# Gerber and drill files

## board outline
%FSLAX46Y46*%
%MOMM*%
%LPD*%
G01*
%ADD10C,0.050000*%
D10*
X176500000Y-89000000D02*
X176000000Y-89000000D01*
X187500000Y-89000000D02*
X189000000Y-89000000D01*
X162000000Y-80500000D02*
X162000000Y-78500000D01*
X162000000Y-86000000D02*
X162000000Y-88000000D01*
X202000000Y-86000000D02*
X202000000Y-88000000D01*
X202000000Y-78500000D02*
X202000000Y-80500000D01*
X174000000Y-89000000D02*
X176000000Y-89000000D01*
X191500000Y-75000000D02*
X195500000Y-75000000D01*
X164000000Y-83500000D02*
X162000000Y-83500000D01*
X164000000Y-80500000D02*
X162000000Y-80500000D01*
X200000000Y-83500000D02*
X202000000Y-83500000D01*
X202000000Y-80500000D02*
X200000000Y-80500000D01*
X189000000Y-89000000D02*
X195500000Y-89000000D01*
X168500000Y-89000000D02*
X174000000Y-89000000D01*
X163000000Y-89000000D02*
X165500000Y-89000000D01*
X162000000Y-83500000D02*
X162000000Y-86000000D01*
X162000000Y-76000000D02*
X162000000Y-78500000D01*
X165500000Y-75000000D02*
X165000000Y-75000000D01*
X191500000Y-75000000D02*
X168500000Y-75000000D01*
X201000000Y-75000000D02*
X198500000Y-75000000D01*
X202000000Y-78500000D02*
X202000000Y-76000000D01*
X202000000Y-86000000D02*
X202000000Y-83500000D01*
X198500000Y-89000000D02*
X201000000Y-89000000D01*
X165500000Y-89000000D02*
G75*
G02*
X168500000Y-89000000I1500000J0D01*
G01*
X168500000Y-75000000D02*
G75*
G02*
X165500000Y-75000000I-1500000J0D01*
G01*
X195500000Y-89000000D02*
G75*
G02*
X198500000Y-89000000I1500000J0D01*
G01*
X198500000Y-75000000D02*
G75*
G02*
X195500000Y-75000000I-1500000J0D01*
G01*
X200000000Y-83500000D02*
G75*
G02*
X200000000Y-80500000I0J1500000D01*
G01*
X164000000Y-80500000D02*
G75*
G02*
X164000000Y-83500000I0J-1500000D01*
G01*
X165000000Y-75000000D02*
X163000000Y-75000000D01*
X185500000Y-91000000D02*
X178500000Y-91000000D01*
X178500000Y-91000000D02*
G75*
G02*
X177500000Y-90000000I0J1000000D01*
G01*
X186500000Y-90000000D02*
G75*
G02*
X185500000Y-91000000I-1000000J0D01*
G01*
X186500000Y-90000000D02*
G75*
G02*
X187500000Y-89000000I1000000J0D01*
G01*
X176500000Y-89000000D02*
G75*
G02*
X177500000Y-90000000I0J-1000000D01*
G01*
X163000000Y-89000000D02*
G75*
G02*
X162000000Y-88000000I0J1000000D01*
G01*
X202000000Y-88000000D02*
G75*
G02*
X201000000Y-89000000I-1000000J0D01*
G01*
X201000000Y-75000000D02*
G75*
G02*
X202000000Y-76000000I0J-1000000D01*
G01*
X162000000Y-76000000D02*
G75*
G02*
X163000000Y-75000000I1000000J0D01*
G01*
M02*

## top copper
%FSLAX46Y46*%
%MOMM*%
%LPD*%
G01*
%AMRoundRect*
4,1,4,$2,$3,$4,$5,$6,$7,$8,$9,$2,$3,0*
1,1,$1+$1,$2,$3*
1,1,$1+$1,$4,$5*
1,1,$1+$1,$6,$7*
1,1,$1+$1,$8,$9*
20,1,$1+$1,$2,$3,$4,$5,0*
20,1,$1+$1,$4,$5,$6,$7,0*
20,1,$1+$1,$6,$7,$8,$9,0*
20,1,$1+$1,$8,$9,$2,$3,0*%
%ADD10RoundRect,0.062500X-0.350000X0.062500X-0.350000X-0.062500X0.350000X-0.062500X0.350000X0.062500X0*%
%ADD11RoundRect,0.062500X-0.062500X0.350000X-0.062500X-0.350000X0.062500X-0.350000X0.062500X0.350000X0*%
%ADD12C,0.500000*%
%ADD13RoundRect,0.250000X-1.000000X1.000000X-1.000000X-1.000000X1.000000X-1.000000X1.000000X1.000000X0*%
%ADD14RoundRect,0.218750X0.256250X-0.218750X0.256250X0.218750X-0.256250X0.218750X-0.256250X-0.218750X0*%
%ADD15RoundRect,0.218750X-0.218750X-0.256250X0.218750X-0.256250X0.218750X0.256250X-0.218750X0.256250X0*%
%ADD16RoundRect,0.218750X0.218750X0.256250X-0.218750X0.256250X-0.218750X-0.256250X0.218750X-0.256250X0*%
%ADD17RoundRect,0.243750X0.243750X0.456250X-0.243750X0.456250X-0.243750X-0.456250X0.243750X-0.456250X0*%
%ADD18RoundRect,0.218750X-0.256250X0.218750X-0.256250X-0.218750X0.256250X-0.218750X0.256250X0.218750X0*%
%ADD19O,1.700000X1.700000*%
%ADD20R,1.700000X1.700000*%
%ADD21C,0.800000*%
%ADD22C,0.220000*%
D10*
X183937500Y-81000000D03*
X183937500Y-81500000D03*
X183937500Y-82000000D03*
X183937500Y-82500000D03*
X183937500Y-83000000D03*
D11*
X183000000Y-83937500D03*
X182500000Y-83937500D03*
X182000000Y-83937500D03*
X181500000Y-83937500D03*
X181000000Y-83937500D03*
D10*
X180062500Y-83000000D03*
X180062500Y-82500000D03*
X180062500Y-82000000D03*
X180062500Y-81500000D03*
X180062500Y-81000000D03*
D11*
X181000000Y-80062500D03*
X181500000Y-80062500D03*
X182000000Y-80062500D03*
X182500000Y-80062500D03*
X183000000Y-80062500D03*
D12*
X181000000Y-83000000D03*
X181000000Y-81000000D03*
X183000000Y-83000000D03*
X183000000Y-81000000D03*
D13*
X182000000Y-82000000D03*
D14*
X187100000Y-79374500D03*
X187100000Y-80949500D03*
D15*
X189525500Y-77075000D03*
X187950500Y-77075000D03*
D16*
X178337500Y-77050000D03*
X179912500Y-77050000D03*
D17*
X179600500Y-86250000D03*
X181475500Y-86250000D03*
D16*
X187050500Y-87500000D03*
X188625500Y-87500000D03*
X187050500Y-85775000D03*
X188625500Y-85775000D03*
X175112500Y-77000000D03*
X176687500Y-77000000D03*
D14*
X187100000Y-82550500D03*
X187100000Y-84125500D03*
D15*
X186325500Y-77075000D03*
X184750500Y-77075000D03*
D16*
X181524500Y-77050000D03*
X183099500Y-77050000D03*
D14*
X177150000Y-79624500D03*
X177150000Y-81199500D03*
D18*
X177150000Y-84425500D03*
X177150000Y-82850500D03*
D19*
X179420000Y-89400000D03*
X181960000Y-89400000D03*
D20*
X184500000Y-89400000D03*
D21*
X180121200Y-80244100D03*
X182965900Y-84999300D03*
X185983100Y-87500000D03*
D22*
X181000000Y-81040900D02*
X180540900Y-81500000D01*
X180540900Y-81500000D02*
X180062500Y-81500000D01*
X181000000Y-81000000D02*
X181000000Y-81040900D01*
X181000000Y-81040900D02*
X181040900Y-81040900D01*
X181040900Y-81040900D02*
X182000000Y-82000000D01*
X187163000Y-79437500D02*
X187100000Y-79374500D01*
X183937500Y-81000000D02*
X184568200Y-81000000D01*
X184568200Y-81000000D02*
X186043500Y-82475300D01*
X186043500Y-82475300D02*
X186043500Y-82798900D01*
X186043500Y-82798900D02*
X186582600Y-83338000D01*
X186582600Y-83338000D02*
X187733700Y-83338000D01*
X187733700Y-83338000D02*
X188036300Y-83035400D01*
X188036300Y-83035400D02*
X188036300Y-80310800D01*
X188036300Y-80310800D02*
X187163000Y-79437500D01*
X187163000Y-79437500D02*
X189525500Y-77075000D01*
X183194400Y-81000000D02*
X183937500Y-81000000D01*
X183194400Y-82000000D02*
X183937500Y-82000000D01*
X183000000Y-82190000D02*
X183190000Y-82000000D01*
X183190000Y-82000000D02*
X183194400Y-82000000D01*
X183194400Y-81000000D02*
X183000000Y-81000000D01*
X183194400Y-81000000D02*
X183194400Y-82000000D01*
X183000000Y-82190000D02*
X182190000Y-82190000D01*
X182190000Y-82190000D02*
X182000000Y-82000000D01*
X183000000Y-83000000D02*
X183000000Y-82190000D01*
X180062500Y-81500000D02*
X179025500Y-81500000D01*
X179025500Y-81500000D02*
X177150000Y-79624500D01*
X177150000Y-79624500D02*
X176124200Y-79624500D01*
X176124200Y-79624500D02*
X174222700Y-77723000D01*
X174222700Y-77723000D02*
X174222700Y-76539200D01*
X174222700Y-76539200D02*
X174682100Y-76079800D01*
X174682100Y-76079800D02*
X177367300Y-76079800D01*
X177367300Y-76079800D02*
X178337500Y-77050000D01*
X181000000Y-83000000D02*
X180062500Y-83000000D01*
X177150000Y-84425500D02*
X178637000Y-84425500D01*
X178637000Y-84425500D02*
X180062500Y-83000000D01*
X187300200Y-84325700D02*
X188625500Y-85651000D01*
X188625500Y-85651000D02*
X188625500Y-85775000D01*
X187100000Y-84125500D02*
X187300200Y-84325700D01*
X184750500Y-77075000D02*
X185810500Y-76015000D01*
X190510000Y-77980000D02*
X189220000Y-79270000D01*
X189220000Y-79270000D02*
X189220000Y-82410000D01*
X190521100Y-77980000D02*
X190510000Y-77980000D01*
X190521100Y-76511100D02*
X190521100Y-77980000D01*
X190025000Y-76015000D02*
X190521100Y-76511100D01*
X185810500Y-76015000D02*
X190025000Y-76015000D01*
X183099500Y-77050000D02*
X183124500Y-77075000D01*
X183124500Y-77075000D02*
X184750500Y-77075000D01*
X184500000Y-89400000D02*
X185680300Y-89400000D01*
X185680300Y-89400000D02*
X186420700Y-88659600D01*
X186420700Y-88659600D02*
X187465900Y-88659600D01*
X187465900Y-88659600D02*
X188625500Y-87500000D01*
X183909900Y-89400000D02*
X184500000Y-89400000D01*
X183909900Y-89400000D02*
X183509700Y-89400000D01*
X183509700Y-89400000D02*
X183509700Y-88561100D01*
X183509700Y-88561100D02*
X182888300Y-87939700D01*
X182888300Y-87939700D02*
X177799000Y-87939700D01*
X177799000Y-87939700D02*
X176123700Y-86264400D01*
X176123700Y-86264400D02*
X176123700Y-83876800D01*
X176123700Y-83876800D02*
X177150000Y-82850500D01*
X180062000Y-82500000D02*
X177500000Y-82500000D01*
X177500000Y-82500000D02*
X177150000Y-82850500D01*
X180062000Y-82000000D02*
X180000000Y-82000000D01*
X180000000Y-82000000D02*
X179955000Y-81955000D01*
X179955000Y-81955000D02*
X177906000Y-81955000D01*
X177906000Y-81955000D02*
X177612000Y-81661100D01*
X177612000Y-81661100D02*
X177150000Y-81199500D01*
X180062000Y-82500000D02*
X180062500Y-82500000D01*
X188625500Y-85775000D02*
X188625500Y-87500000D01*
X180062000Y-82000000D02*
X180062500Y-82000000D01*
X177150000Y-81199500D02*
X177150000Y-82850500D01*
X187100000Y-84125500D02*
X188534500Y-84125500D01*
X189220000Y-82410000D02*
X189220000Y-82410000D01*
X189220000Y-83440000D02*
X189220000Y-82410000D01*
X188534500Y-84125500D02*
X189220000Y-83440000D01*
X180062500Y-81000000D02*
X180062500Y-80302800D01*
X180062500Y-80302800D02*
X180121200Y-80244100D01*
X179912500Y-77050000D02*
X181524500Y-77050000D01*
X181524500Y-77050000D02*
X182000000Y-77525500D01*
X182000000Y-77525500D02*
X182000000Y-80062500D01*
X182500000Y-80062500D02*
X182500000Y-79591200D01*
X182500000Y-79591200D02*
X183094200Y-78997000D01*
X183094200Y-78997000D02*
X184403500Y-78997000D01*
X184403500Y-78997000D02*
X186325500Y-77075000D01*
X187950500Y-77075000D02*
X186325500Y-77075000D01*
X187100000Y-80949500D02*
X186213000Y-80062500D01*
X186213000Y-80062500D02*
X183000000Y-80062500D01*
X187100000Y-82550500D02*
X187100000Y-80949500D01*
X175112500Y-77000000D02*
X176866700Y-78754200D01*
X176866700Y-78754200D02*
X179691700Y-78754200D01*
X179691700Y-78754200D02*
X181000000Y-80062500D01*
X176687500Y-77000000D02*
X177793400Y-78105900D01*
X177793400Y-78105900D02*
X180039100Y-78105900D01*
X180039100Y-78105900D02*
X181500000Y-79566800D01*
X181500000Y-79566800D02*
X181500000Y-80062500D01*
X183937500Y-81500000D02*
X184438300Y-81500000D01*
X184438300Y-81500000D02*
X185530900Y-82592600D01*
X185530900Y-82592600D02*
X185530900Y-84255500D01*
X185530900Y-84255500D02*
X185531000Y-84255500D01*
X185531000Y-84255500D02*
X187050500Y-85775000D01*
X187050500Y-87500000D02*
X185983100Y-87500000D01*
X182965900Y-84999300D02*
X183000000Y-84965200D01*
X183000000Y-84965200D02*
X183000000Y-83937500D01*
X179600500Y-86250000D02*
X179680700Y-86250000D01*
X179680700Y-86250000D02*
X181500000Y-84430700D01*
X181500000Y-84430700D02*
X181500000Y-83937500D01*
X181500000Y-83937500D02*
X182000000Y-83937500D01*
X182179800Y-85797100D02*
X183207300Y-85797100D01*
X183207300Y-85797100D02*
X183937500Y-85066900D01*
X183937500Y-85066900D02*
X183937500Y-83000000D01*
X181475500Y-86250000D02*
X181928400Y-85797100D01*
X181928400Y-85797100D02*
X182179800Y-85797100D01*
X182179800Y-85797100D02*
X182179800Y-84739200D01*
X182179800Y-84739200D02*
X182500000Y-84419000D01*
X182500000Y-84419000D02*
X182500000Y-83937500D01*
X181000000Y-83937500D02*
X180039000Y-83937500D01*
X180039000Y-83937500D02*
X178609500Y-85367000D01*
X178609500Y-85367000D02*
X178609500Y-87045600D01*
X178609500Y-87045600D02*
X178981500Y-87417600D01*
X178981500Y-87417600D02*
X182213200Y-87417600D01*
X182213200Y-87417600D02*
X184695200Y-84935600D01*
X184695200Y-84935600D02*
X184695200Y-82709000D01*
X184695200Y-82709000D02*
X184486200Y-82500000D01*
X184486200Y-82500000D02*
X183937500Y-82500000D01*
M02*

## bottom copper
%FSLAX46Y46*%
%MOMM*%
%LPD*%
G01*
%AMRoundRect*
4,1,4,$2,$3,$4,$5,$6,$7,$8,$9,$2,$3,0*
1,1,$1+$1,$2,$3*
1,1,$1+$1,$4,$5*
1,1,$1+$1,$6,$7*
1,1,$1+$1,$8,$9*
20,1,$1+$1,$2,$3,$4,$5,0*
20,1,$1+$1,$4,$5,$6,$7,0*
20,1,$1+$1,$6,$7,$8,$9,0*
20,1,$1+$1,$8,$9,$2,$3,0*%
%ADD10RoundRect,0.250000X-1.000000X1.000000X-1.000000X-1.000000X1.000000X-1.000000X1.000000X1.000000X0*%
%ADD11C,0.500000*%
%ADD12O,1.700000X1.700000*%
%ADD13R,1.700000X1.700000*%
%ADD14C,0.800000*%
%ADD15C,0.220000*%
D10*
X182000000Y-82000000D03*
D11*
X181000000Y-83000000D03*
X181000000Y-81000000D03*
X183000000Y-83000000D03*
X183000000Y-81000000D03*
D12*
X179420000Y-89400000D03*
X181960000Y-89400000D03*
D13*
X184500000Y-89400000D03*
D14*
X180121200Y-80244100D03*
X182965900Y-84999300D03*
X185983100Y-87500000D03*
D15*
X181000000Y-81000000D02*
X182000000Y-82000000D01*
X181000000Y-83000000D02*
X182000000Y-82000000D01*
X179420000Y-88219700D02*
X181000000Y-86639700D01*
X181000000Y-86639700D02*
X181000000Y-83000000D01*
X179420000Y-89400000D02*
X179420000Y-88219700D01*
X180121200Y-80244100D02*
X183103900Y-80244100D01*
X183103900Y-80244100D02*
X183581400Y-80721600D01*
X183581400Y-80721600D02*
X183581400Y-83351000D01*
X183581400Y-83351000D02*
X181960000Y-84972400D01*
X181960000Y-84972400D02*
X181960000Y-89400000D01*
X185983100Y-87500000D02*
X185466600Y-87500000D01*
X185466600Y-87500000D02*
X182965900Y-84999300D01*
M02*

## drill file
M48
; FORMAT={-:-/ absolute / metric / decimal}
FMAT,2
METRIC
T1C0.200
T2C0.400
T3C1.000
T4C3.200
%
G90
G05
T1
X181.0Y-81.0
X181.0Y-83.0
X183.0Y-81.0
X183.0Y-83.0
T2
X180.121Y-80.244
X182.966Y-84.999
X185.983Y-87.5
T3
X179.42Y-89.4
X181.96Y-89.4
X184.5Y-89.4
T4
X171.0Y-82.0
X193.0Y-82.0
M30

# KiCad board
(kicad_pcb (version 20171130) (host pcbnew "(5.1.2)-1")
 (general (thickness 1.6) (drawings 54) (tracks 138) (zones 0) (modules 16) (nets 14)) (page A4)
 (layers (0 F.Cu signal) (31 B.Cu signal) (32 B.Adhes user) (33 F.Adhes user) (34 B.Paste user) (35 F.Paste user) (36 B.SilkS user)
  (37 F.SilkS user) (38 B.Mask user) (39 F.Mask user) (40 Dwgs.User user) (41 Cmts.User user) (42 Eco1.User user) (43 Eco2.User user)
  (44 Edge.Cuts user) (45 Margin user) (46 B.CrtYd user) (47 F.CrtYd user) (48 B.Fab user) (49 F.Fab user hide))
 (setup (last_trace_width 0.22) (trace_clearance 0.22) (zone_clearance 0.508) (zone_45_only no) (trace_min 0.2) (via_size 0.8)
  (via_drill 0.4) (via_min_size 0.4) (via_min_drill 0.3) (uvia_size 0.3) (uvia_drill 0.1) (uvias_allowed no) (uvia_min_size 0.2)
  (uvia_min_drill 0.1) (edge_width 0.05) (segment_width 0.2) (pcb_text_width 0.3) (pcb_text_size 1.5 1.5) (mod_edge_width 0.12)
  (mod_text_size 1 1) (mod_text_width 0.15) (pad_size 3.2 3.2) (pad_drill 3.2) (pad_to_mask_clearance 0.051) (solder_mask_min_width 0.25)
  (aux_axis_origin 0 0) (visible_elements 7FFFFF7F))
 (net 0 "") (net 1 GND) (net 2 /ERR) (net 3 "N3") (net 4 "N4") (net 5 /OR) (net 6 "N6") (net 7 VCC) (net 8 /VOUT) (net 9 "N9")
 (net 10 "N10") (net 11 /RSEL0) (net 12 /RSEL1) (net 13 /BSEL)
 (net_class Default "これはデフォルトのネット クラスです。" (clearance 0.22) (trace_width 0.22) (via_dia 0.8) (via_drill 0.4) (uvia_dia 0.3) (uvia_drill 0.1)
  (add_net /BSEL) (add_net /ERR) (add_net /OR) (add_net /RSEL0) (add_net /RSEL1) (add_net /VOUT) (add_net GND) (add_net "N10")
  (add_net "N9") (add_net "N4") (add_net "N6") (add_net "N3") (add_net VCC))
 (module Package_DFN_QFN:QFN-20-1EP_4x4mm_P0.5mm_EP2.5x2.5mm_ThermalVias (layer F.Cu) (at 182 82 270)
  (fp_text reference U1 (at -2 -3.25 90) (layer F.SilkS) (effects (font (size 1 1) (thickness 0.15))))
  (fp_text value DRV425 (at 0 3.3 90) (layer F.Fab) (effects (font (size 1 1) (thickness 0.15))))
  (pad 20 smd roundrect (at -1 -1.9375 270) (size 0.25 0.825) (layers F.Cu F.Paste F.Mask) (roundrect_rratio 0.25) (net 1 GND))
  (pad 19 smd roundrect (at -0.5 -1.9375 270) (size 0.25 0.825) (layers F.Cu F.Paste F.Mask) (roundrect_rratio 0.25) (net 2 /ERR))
  (pad 18 smd roundrect (at 0 -1.9375 270) (size 0.25 0.825) (layers F.Cu F.Paste F.Mask) (roundrect_rratio 0.25) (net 1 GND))
  (pad 17 smd roundrect (at 0.5 -1.9375 270) (size 0.25 0.825) (layers F.Cu F.Paste F.Mask) (roundrect_rratio 0.25) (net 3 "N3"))
  (pad 16 smd roundrect (at 1 -1.9375 270) (size 0.25 0.825) (layers F.Cu F.Paste F.Mask) (roundrect_rratio 0.25) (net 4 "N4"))
  (pad 15 smd roundrect (at 1.9375 -1 270) (size 0.825 0.25) (layers F.Cu F.Paste F.Mask) (roundrect_rratio 0.25) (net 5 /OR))
  (pad 14 smd roundrect (at 1.9375 -0.5 270) (size 0.825 0.25) (layers F.Cu F.Paste F.Mask) (roundrect_rratio 0.25) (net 4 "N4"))
  (pad 13 smd roundrect (at 1.9375 0 270) (size 0.825 0.25) (layers F.Cu F.Paste F.Mask) (roundrect_rratio 0.25) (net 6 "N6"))
  (pad 12 smd roundrect (at 1.9375 0.5 270) (size 0.825 0.25) (layers F.Cu F.Paste F.Mask) (roundrect_rratio 0.25) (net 6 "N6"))
  (pad 11 smd roundrect (at 1.9375 1 270) (size 0.825 0.25) (layers F.Cu F.Paste F.Mask) (roundrect_rratio 0.25) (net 3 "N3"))
  (pad 10 smd roundrect (at 1 1.9375 270) (size 0.25 0.825) (layers F.Cu F.Paste F.Mask) (roundrect_rratio 0.25) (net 1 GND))
  (pad 9 smd roundrect (at 0.5 1.9375 270) (size 0.25 0.825) (layers F.Cu F.Paste F.Mask) (roundrect_rratio 0.25) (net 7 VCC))
  (pad 8 smd roundrect (at 0 1.9375 270) (size 0.25 0.825) (layers F.Cu F.Paste F.Mask) (roundrect_rratio 0.25) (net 7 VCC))
  (pad 7 smd roundrect (at -0.5 1.9375 270) (size 0.25 0.825) (layers F.Cu F.Paste F.Mask) (roundrect_rratio 0.25) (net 1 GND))
  (pad 6 smd roundrect (at -1 1.9375 270) (size 0.25 0.825) (layers F.Cu F.Paste F.Mask) (roundrect_rratio 0.25) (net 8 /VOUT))
  (pad 5 smd roundrect (at -1.9375 1 270) (size 0.825 0.25) (layers F.Cu F.Paste F.Mask) (roundrect_rratio 0.25) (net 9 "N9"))
  (pad 4 smd roundrect (at -1.9375 0.5 270) (size 0.825 0.25) (layers F.Cu F.Paste F.Mask) (roundrect_rratio 0.25) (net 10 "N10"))
  (pad 3 smd roundrect (at -1.9375 0 270) (size 0.825 0.25) (layers F.Cu F.Paste F.Mask) (roundrect_rratio 0.25) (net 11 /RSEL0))
  (pad 2 smd roundrect (at -1.9375 -0.5 270) (size 0.825 0.25) (layers F.Cu F.Paste F.Mask) (roundrect_rratio 0.25) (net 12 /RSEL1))
  (pad 1 smd roundrect (at -1.9375 -1 270) (size 0.825 0.25) (layers F.Cu F.Paste F.Mask) (roundrect_rratio 0.25) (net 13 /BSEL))
  (pad "" smd roundrect (at 0.625 0.625 270) (size 1.08 1.08) (layers F.Paste) (roundrect_rratio 0.231481))
  (pad "" smd roundrect (at 0.625 -0.625 270) (size 1.08 1.08) (layers F.Paste) (roundrect_rratio 0.231481))
  (pad "" smd roundrect (at -0.625 0.625 270) (size 1.08 1.08) (layers F.Paste) (roundrect_rratio 0.231481))
  (pad "" smd roundrect (at -0.625 -0.625 270) (size 1.08 1.08) (layers F.Paste) (roundrect_rratio 0.231481))
  (pad 21 smd roundrect (at 0 0 270) (size 2.5 2.5) (layers B.Cu) (roundrect_rratio 0.1) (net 1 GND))
  (pad 21 thru_hole circle (at 1 1 270) (size 0.5 0.5) (drill 0.2) (layers *.Cu) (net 1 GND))
  (pad 21 thru_hole circle (at -1 1 270) (size 0.5 0.5) (drill 0.2) (layers *.Cu) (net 1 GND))
  (pad 21 thru_hole circle (at 1 -1 270) (size 0.5 0.5) (drill 0.2) (layers *.Cu) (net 1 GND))
  (pad 21 thru_hole circle (at -1 -1 270) (size 0.5 0.5) (drill 0.2) (layers *.Cu) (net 1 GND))
  (pad 21 smd roundrect (at 0 0 270) (size 2.5 2.5) (layers F.Cu F.Mask) (roundrect_rratio 0.1) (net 1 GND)))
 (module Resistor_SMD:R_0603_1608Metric (layer F.Cu) (at 187.1 80.162 90)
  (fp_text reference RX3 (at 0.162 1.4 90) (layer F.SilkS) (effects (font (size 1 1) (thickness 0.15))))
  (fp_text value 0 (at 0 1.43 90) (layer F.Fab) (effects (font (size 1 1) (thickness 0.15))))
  (pad 2 smd roundrect (at 0.7875 0 90) (size 0.875 0.95) (layers F.Cu F.Paste F.Mask) (roundrect_rratio 0.25) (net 1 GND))
  (pad 1 smd roundrect (at -0.7875 0 90) (size 0.875 0.95) (layers F.Cu F.Paste F.Mask) (roundrect_rratio 0.25) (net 13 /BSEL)))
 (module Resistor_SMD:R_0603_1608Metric (layer F.Cu) (at 188.738 77.075)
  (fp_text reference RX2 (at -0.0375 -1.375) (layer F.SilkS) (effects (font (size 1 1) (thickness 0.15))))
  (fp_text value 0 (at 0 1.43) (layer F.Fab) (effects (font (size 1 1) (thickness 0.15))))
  (pad 2 smd roundrect (at 0.7875 0) (size 0.875 0.95) (layers F.Cu F.Paste F.Mask) (roundrect_rratio 0.25) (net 1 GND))
  (pad 1 smd roundrect (at -0.7875 0) (size 0.875 0.95) (layers F.Cu F.Paste F.Mask) (roundrect_rratio 0.25) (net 12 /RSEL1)))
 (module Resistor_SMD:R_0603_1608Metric (layer F.Cu) (at 179.125 77.05 180)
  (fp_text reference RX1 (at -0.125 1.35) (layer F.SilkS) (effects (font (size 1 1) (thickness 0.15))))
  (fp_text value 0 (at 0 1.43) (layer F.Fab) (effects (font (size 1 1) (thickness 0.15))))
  (pad 2 smd roundrect (at 0.7875 0 180) (size 0.875 0.95) (layers F.Cu F.Paste F.Mask) (roundrect_rratio 0.25) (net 1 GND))
  (pad 1 smd roundrect (at -0.7875 0 180) (size 0.875 0.95) (layers F.Cu F.Paste F.Mask) (roundrect_rratio 0.25) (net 11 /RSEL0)))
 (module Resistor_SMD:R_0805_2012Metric (layer F.Cu) (at 180.538 86.25 180)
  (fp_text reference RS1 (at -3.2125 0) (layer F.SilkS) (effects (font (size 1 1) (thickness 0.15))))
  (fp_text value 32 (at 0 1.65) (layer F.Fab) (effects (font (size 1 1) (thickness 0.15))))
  (pad 2 smd roundrect (at 0.9375 0 180) (size 0.975 1.4) (layers F.Cu F.Paste F.Mask) (roundrect_rratio 0.25) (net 6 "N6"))
  (pad 1 smd roundrect (at -0.9375 0 180) (size 0.975 1.4) (layers F.Cu F.Paste F.Mask) (roundrect_rratio 0.25) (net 4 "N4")))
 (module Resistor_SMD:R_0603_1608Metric (layer F.Cu) (at 187.838 87.5 180)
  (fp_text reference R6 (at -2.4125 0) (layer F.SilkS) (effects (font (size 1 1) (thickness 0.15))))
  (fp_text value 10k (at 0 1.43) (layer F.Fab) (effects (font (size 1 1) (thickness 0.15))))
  (pad 2 smd roundrect (at 0.7875 0 180) (size 0.875 0.95) (layers F.Cu F.Paste F.Mask) (roundrect_rratio 0.25) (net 5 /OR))
  (pad 1 smd roundrect (at -0.7875 0 180) (size 0.875 0.95) (layers F.Cu F.Paste F.Mask) (roundrect_rratio 0.25) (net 7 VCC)))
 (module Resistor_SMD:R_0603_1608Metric (layer F.Cu) (at 187.838 85.775 180)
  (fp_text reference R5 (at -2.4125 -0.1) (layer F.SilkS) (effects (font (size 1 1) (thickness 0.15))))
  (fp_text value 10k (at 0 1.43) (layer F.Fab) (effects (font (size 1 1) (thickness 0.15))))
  (pad 2 smd roundrect (at 0.7875 0 180) (size 0.875 0.95) (layers F.Cu F.Paste F.Mask) (roundrect_rratio 0.25) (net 2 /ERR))
  (pad 1 smd roundrect (at -0.7875 0 180) (size 0.875 0.95) (layers F.Cu F.Paste F.Mask) (roundrect_rratio 0.25) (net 7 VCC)))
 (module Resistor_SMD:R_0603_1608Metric (layer F.Cu) (at 175.9 77 180)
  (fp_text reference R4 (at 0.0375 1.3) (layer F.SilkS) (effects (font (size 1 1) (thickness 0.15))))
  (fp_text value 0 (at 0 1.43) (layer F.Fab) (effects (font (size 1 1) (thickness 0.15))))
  (pad 2 smd roundrect (at 0.7875 0 180) (size 0.875 0.95) (layers F.Cu F.Paste F.Mask) (roundrect_rratio 0.25) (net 9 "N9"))
  (pad 1 smd roundrect (at -0.7875 0 180) (size 0.875 0.95) (layers F.Cu F.Paste F.Mask) (roundrect_rratio 0.25) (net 10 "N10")))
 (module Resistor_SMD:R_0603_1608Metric (layer F.Cu) (at 187.1 83.338 90)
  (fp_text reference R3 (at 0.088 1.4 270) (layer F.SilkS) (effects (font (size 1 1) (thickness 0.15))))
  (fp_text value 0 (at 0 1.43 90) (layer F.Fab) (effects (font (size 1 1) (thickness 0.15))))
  (pad 2 smd roundrect (at 0.7875 0 90) (size 0.875 0.95) (layers F.Cu F.Paste F.Mask) (roundrect_rratio 0.25) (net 13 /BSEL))
  (pad 1 smd roundrect (at -0.7875 0 90) (size 0.875 0.95) (layers F.Cu F.Paste F.Mask) (roundrect_rratio 0.25) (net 7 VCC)))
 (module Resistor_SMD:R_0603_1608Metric (layer F.Cu) (at 185.538 77.075)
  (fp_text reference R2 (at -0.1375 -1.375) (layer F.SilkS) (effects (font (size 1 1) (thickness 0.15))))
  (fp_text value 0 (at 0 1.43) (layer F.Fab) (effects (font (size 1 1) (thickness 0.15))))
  (pad 2 smd roundrect (at 0.7875 0) (size 0.875 0.95) (layers F.Cu F.Paste F.Mask) (roundrect_rratio 0.25) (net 12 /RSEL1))
  (pad 1 smd roundrect (at -0.7875 0) (size 0.875 0.95) (layers F.Cu F.Paste F.Mask) (roundrect_rratio 0.25) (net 7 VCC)))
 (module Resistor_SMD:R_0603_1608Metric (layer F.Cu) (at 182.312 77.05 180)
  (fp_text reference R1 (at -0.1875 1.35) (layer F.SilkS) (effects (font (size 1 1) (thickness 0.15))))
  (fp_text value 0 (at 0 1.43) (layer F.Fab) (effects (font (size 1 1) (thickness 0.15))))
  (pad 2 smd roundrect (at 0.7875 0 180) (size 0.875 0.95) (layers F.Cu F.Paste F.Mask) (roundrect_rratio 0.25) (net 11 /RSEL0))
  (pad 1 smd roundrect (at -0.7875 0 180) (size 0.875 0.95) (layers F.Cu F.Paste F.Mask) (roundrect_rratio 0.25) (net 7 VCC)))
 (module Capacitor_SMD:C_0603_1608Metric (layer F.Cu) (at 177.15 80.412 90)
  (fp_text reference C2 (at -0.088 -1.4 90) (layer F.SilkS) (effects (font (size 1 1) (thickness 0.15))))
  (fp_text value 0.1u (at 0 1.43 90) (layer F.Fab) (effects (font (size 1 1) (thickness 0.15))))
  (pad 2 smd roundrect (at 0.7875 0 90) (size 0.875 0.95) (layers F.Cu F.Paste F.Mask) (roundrect_rratio 0.25) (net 1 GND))
  (pad 1 smd roundrect (at -0.7875 0 90) (size 0.875 0.95) (layers F.Cu F.Paste F.Mask) (roundrect_rratio 0.25) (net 7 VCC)))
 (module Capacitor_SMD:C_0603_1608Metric (layer F.Cu) (at 177.15 83.638 270)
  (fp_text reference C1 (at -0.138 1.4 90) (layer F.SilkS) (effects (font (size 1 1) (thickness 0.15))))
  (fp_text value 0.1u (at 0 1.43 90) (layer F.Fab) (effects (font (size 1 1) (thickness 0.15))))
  (pad 2 smd roundrect (at 0.7875 0 270) (size 0.875 0.95) (layers F.Cu F.Paste F.Mask) (roundrect_rratio 0.25) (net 1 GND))
  (pad 1 smd roundrect (at -0.7875 0 270) (size 0.875 0.95) (layers F.Cu F.Paste F.Mask) (roundrect_rratio 0.25) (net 7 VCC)))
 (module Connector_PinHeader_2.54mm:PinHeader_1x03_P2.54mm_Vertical (layer F.Cu) (at 184.5 89.4 270)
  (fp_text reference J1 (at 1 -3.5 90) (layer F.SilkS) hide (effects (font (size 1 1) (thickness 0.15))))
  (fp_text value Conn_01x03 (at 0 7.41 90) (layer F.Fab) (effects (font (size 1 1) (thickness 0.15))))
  (pad 3 thru_hole oval (at 0 5.08 270) (size 1.7 1.7) (drill 1) (layers *.Cu *.Mask) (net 1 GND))
  (pad 2 thru_hole oval (at 0 2.54 270) (size 1.7 1.7) (drill 1) (layers *.Cu *.Mask) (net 8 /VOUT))
  (pad 1 thru_hole rect (at 0 0 270) (size 1.7 1.7) (drill 1) (layers *.Cu *.Mask) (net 7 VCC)))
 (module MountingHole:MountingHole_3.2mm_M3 (layer F.Cu) (at 171 82)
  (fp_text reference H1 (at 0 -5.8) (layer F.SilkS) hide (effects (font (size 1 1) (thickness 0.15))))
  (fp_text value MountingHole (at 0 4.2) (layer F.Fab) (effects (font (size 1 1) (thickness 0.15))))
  (pad "" np_thru_hole circle (at 0 0) (size 3.2 3.2) (drill 3.2) (layers *.Cu)))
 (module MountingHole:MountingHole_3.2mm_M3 (layer F.Cu) (at 193 82)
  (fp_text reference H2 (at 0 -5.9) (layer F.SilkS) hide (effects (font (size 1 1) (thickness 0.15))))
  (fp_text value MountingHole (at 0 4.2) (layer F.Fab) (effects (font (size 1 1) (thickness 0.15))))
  (pad "" np_thru_hole circle (at 0 0) (size 3.2 3.2) (drill 3.2) (layers *.Cu)))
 (gr_line (start 176.5 89) (end 176 89) (layer Edge.Cuts) (width 0.05))
 (gr_line (start 187.5 89) (end 189 89) (layer Edge.Cuts) (width 0.05))
 (gr_line (start 162 80.5) (end 162 78.5) (layer Edge.Cuts) (width 0.05))
 (gr_line (start 162 86) (end 162 88) (layer Edge.Cuts) (width 0.05))
 (gr_line (start 202 86) (end 202 88) (layer Edge.Cuts) (width 0.05))
 (gr_line (start 202 78.5) (end 202 80.5) (layer Edge.Cuts) (width 0.05))
 (gr_line (start 174 89) (end 176 89) (layer Edge.Cuts) (width 0.05))
 (gr_line (start 191.5 75) (end 195.5 75) (layer Edge.Cuts) (width 0.05))
 (gr_line (start 164 83.5) (end 162 83.5) (layer Edge.Cuts) (width 0.05))
 (gr_line (start 164 80.5) (end 162 80.5) (layer Edge.Cuts) (width 0.05))
 (gr_line (start 200 83.5) (end 202 83.5) (layer Edge.Cuts) (width 0.05))
 (gr_line (start 202 80.5) (end 200 80.5) (layer Edge.Cuts) (width 0.05))
 (gr_line (start 189 89) (end 195.5 89) (layer Edge.Cuts) (width 0.05))
 (gr_line (start 168.5 89) (end 174 89) (layer Edge.Cuts) (width 0.05))
 (gr_line (start 163 89) (end 165.5 89) (layer Edge.Cuts) (width 0.05))
 (gr_line (start 162 83.5) (end 162 86) (layer Edge.Cuts) (width 0.05))
 (gr_line (start 162 76) (end 162 78.5) (layer Edge.Cuts) (width 0.05))
 (gr_line (start 165.5 75) (end 165 75) (layer Edge.Cuts) (width 0.05))
 (gr_line (start 191.5 75) (end 168.5 75) (layer Edge.Cuts) (width 0.05))
 (gr_line (start 201 75) (end 198.5 75) (layer Edge.Cuts) (width 0.05))
 (gr_line (start 202 78.5) (end 202 76) (layer Edge.Cuts) (width 0.05))
 (gr_line (start 202 86) (end 202 83.5) (layer Edge.Cuts) (width 0.05))
 (gr_line (start 198.5 89) (end 201 89) (layer Edge.Cuts) (width 0.05))
 (gr_arc (start 167 89) (end 168.5 89) (angle -180) (layer Edge.Cuts) (width 0.05))
 (gr_arc (start 167 75) (end 165.5 75) (angle -180) (layer Edge.Cuts) (width 0.05))
 (gr_arc (start 197 89) (end 198.5 89) (angle -180) (layer Edge.Cuts) (width 0.05))
 (gr_arc (start 197 75) (end 195.5 75) (angle -180) (layer Edge.Cuts) (width 0.05))
 (gr_arc (start 200 82) (end 200 80.5) (angle -180) (layer Edge.Cuts) (width 0.05))
 (gr_arc (start 164 82) (end 164 83.5) (angle -180) (layer Edge.Cuts) (width 0.05))
 (gr_line (start 165 75) (end 163 75) (layer Edge.Cuts) (width 0.05))
 (gr_line (start 185.5 91) (end 178.5 91) (layer Edge.Cuts) (width 0.05))
 (gr_arc (start 178.5 90) (end 177.5 90) (angle -90) (layer Edge.Cuts) (width 0.05))
 (gr_arc (start 185.5 90) (end 185.5 91) (angle -90) (layer Edge.Cuts) (width 0.05))
 (gr_arc (start 187.5 90) (end 187.5 89) (angle -90) (layer Edge.Cuts) (width 0.05))
 (gr_arc (start 176.5 90) (end 177.5 90) (angle -90) (layer Edge.Cuts) (width 0.05))
 (gr_arc (start 163 88) (end 162 88) (angle -90) (layer Edge.Cuts) (width 0.05))
 (gr_arc (start 201 88) (end 201 89) (angle -90) (layer Edge.Cuts) (width 0.05))
 (gr_arc (start 201 76) (end 202 76) (angle -90) (layer Edge.Cuts) (width 0.05))
 (gr_arc (start 163 76) (end 163 75) (angle -90) (layer Edge.Cuts) (width 0.05))
 (segment (start 181 81.0409) (end 180.5409 81.5) (width 0.22) (layer F.Cu) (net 1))
 (segment (start 180.5409 81.5) (end 180.0625 81.5) (width 0.22) (layer F.Cu) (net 1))
 (segment (start 181 81) (end 181 81.0409) (width 0.22) (layer F.Cu) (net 1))
 (segment (start 181 81.0409) (end 181.0409 81.0409) (width 0.22) (layer F.Cu) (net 1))
 (segment (start 181.0409 81.0409) (end 182 82) (width 0.22) (layer F.Cu) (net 1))
 (segment (start 187.163 79.4375) (end 187.1 79.3745) (width 0.22) (layer F.Cu) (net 1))
 (segment (start 183.9375 81) (end 184.5682 81) (width 0.22) (layer F.Cu) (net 1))
 (segment (start 184.5682 81) (end 186.0435 82.4753) (width 0.22) (layer F.Cu) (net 1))
 (segment (start 186.0435 82.4753) (end 186.0435 82.7989) (width 0.22) (layer F.Cu) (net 1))
 (segment (start 186.0435 82.7989) (end 186.5826 83.338) (width 0.22) (layer F.Cu) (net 1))
 (segment (start 186.5826 83.338) (end 187.7337 83.338) (width 0.22) (layer F.Cu) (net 1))
 (segment (start 187.7337 83.338) (end 188.0363 83.0354) (width 0.22) (layer F.Cu) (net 1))
 (segment (start 188.0363 83.0354) (end 188.0363 80.3108) (width 0.22) (layer F.Cu) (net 1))
 (segment (start 188.0363 80.3108) (end 187.163 79.4375) (width 0.22) (layer F.Cu) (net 1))
 (segment (start 187.163 79.4375) (end 189.5255 77.075) (width 0.22) (layer F.Cu) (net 1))
 (segment (start 183.1944 81) (end 183.9375 81) (width 0.22) (layer F.Cu) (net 1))
 (segment (start 183.1944 82) (end 183.9375 82) (width 0.22) (layer F.Cu) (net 1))
 (segment (start 183 82.19) (end 183.19 82) (width 0.22) (layer F.Cu) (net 1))
 (segment (start 183.19 82) (end 183.1944 82) (width 0.22) (layer F.Cu) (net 1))
 (segment (start 183.1944 81) (end 183 81) (width 0.22) (layer F.Cu) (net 1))
 (segment (start 183.1944 81) (end 183.1944 82) (width 0.22) (layer F.Cu) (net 1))
 (segment (start 183 82.19) (end 182.19 82.19) (width 0.22) (layer F.Cu) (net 1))
 (segment (start 182.19 82.19) (end 182 82) (width 0.22) (layer F.Cu) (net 1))
 (segment (start 183 83) (end 183 82.19) (width 0.22) (layer F.Cu) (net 1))
 (segment (start 180.0625 81.5) (end 179.0255 81.5) (width 0.22) (layer F.Cu) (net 1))
 (segment (start 179.0255 81.5) (end 177.15 79.6245) (width 0.22) (layer F.Cu) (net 1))
 (segment (start 177.15 79.6245) (end 176.1242 79.6245) (width 0.22) (layer F.Cu) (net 1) (status 400000))
 (segment (start 176.1242 79.6245) (end 174.2227 77.723) (width 0.22) (layer F.Cu) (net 1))
 (segment (start 174.2227 77.723) (end 174.2227 76.5392) (width 0.22) (layer F.Cu) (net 1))
 (segment (start 174.2227 76.5392) (end 174.6821 76.0798) (width 0.22) (layer F.Cu) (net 1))
 (segment (start 174.6821 76.0798) (end 177.3673 76.0798) (width 0.22) (layer F.Cu) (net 1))
 (segment (start 177.3673 76.0798) (end 178.3375 77.05) (width 0.22) (layer F.Cu) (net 1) (status 800000))
 (segment (start 181 81) (end 182 82) (width 0.22) (layer B.Cu) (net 1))
 (segment (start 181 83) (end 182 82) (width 0.22) (layer B.Cu) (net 1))
 (segment (start 179.42 88.2197) (end 181 86.6397) (width 0.22) (layer B.Cu) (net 1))
 (segment (start 181 86.6397) (end 181 83) (width 0.22) (layer B.Cu) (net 1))
 (segment (start 181 83) (end 180.0625 83) (width 0.22) (layer F.Cu) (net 1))
 (segment (start 177.15 84.4255) (end 178.637 84.4255) (width 0.22) (layer F.Cu) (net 1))
 (segment (start 178.637 84.4255) (end 180.0625 83) (width 0.22) (layer F.Cu) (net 1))
 (segment (start 179.42 89.4) (end 179.42 88.2197) (width 0.22) (layer B.Cu) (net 1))
 (segment (start 187.3002 84.3257) (end 188.6255 85.651) (width 0.22) (layer F.Cu) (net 7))
 (segment (start 188.6255 85.651) (end 188.6255 85.775) (width 0.22) (layer F.Cu) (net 7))
 (segment (start 187.1 84.1255) (end 187.3002 84.3257) (width 0.22) (layer F.Cu) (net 7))
 (segment (start 184.7505 77.075) (end 185.8105 76.015) (width 0.22) (layer F.Cu) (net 7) (status 400000))
 (segment (start 190.51 77.98) (end 189.22 79.27) (width 0.22) (layer F.Cu) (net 7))
 (segment (start 189.22 79.27) (end 189.22 82.41) (width 0.22) (layer F.Cu) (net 7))
 (segment (start 190.5211 77.98) (end 190.51 77.98) (width 0.22) (layer F.Cu) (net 7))
 (segment (start 190.5211 76.5111) (end 190.5211 77.98) (width 0.22) (layer F.Cu) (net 7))
 (segment (start 190.025 76.015) (end 190.5211 76.5111) (width 0.22) (layer F.Cu) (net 7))
 (segment (start 185.8105 76.015) (end 190.025 76.015) (width 0.22) (layer F.Cu) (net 7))
 (segment (start 183.0995 77.05) (end 183.1245 77.075) (width 0.22) (layer F.Cu) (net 7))
 (segment (start 183.1245 77.075) (end 184.7505 77.075) (width 0.22) (layer F.Cu) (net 7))
 (segment (start 184.5 89.4) (end 185.6803 89.4) (width 0.22) (layer F.Cu) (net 7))
 (segment (start 185.6803 89.4) (end 186.4207 88.6596) (width 0.22) (layer F.Cu) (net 7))
 (segment (start 186.4207 88.6596) (end 187.4659 88.6596) (width 0.22) (layer F.Cu) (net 7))
 (segment (start 187.4659 88.6596) (end 188.6255 87.5) (width 0.22) (layer F.Cu) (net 7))
 (segment (start 183.9099 89.4) (end 184.5 89.4) (width 0.22) (layer F.Cu) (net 7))
 (segment (start 183.9099 89.4) (end 183.5097 89.4) (width 0.22) (layer F.Cu) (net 7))
 (segment (start 183.5097 89.4) (end 183.5097 88.5611) (width 0.22) (layer F.Cu) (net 7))
 (segment (start 183.5097 88.5611) (end 182.8883 87.9397) (width 0.22) (layer F.Cu) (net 7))
 (segment (start 182.8883 87.9397) (end 177.799 87.9397) (width 0.22) (layer F.Cu) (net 7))
 (segment (start 177.799 87.9397) (end 176.1237 86.2644) (width 0.22) (layer F.Cu) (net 7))
 (segment (start 176.1237 86.2644) (end 176.1237 83.8768) (width 0.22) (layer F.Cu) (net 7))
 (segment (start 176.1237 83.8768) (end 177.15 82.8505) (width 0.22) (layer F.Cu) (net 7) (status 800000))
 (segment (start 180.062 82.5) (end 177.5 82.5) (width 0.22) (layer F.Cu) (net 7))
 (segment (start 177.5 82.5) (end 177.15 82.8505) (width 0.22) (layer F.Cu) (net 7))
 (segment (start 180.062 82) (end 180 82) (width 0.22) (layer F.Cu) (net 7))
 (segment (start 180 82) (end 179.955 81.955) (width 0.22) (layer F.Cu) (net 7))
 (segment (start 179.955 81.955) (end 177.906 81.955) (width 0.22) (layer F.Cu) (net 7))
 (segment (start 177.906 81.955) (end 177.612 81.6611) (width 0.22) (layer F.Cu) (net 7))
 (segment (start 177.612 81.6611) (end 177.15 81.1995) (width 0.22) (layer F.Cu) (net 7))
 (segment (start 180.062 82.5) (end 180.0625 82.5) (width 0.22) (layer F.Cu) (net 7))
 (segment (start 188.6255 85.775) (end 188.6255 87.5) (width 0.22) (layer F.Cu) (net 7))
 (segment (start 180.062 82) (end 180.0625 82) (width 0.22) (layer F.Cu) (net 7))
 (segment (start 177.15 81.1995) (end 177.15 82.8505) (width 0.22) (layer F.Cu) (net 7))
 (segment (start 187.1 84.1255) (end 188.5345 84.1255) (width 0.22) (layer F.Cu) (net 7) (status 400000))
 (segment (start 189.22 82.41) (end 189.22 82.41) (width 0.22) (layer F.Cu) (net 7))
 (segment (start 189.22 83.44) (end 189.22 82.41) (width 0.22) (layer F.Cu) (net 7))
 (segment (start 188.5345 84.1255) (end 189.22 83.44) (width 0.22) (layer F.Cu) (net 7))
 (segment (start 180.1212 80.2441) (end 183.1039 80.2441) (width 0.22) (layer B.Cu) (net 8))
 (segment (start 183.1039 80.2441) (end 183.5814 80.7216) (width 0.22) (layer B.Cu) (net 8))
 (segment (start 183.5814 80.7216) (end 183.5814 83.351) (width 0.22) (layer B.Cu) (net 8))
 (segment (start 183.5814 83.351) (end 181.96 84.9724) (width 0.22) (layer B.Cu) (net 8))
 (segment (start 181.96 84.9724) (end 181.96 89.4) (width 0.22) (layer B.Cu) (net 8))
 (segment (start 180.0625 81) (end 180.0625 80.3028) (width 0.22) (layer F.Cu) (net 8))
 (segment (start 180.0625 80.3028) (end 180.1212 80.2441) (width 0.22) (layer F.Cu) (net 8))
 (via (at 180.1212 80.2441) (size 0.8) (layers F.Cu B.Cu) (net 8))
 (segment (start 179.9125 77.05) (end 181.5245 77.05) (width 0.22) (layer F.Cu) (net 11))
 (segment (start 181.5245 77.05) (end 182 77.5255) (width 0.22) (layer F.Cu) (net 11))
 (segment (start 182 77.5255) (end 182 80.0625) (width 0.22) (layer F.Cu) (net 11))
 (segment (start 182.5 80.0625) (end 182.5 79.5912) (width 0.22) (layer F.Cu) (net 12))
 (segment (start 182.5 79.5912) (end 183.0942 78.997) (width 0.22) (layer F.Cu) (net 12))
 (segment (start 183.0942 78.997) (end 184.4035 78.997) (width 0.22) (layer F.Cu) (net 12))
 (segment (start 184.4035 78.997) (end 186.3255 77.075) (width 0.22) (layer F.Cu) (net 12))
 (segment (start 187.9505 77.075) (end 186.3255 77.075) (width 0.22) (layer F.Cu) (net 12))
 (segment (start 187.1 80.9495) (end 186.213 80.0625) (width 0.22) (layer F.Cu) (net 13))
 (segment (start 186.213 80.0625) (end 183 80.0625) (width 0.22) (layer F.Cu) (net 13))
 (segment (start 187.1 82.5505) (end 187.1 80.9495) (width 0.22) (layer F.Cu) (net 13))
 (segment (start 175.1125 77) (end 176.8667 78.7542) (width 0.22) (layer F.Cu) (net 9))
 (segment (start 176.8667 78.7542) (end 179.6917 78.7542) (width 0.22) (layer F.Cu) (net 9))
 (segment (start 179.6917 78.7542) (end 181 80.0625) (width 0.22) (layer F.Cu) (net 9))
 (segment (start 176.6875 77) (end 177.7934 78.1059) (width 0.22) (layer F.Cu) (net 10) (status 400000))
 (segment (start 177.7934 78.1059) (end 180.0391 78.1059) (width 0.22) (layer F.Cu) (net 10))
 (segment (start 180.0391 78.1059) (end 181.5 79.5668) (width 0.22) (layer F.Cu) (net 10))
 (segment (start 181.5 79.5668) (end 181.5 80.0625) (width 0.22) (layer F.Cu) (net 10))
 (segment (start 183.9375 81.5) (end 184.4383 81.5) (width 0.22) (layer F.Cu) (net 2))
 (segment (start 184.4383 81.5) (end 185.5309 82.5926) (width 0.22) (layer F.Cu) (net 2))
 (segment (start 185.5309 82.5926) (end 185.5309 84.2555) (width 0.22) (layer F.Cu) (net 2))
 (segment (start 185.5309 84.2555) (end 185.531 84.2555) (width 0.22) (layer F.Cu) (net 2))
 (segment (start 185.531 84.2555) (end 187.0505 85.775) (width 0.22) (layer F.Cu) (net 2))
 (segment (start 187.0505 87.5) (end 185.9831 87.5) (width 0.22) (layer F.Cu) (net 5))
 (segment (start 182.9659 84.9993) (end 183 84.9652) (width 0.22) (layer F.Cu) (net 5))
 (segment (start 183 84.9652) (end 183 83.9375) (width 0.22) (layer F.Cu) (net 5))
 (via (at 182.9659 84.9993) (size 0.8) (layers F.Cu B.Cu) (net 5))
 (via (at 185.9831 87.5) (size 0.8) (layers F.Cu B.Cu) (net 5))
 (segment (start 185.9831 87.5) (end 185.4666 87.5) (width 0.22) (layer B.Cu) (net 5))
 (segment (start 185.4666 87.5) (end 182.9659 84.9993) (width 0.22) (layer B.Cu) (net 5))
 (segment (start 179.6005 86.25) (end 179.6807 86.25) (width 0.22) (layer F.Cu) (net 6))
 (segment (start 179.6807 86.25) (end 181.5 84.4307) (width 0.22) (layer F.Cu) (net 6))
 (segment (start 181.5 84.4307) (end 181.5 83.9375) (width 0.22) (layer F.Cu) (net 6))
 (segment (start 181.5 83.9375) (end 182 83.9375) (width 0.22) (layer F.Cu) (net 6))
 (segment (start 182.1798 85.7971) (end 183.2073 85.7971) (width 0.22) (layer F.Cu) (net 4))
 (segment (start 183.2073 85.7971) (end 183.9375 85.0669) (width 0.22) (layer F.Cu) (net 4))
 (segment (start 183.9375 85.0669) (end 183.9375 83) (width 0.22) (layer F.Cu) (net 4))
 (segment (start 181.4755 86.25) (end 181.9284 85.7971) (width 0.22) (layer F.Cu) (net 4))
 (segment (start 181.9284 85.7971) (end 182.1798 85.7971) (width 0.22) (layer F.Cu) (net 4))
 (segment (start 182.1798 85.7971) (end 182.1798 84.7392) (width 0.22) (layer F.Cu) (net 4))
 (segment (start 182.1798 84.7392) (end 182.5 84.419) (width 0.22) (layer F.Cu) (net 4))
 (segment (start 182.5 84.419) (end 182.5 83.9375) (width 0.22) (layer F.Cu) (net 4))
 (segment (start 181 83.9375) (end 180.039 83.9375) (width 0.22) (layer F.Cu) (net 3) (status 400000))
 (segment (start 180.039 83.9375) (end 178.6095 85.367) (width 0.22) (layer F.Cu) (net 3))
 (segment (start 178.6095 85.367) (end 178.6095 87.0456) (width 0.22) (layer F.Cu) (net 3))
 (segment (start 178.6095 87.0456) (end 178.9815 87.4176) (width 0.22) (layer F.Cu) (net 3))
 (segment (start 178.9815 87.4176) (end 182.2132 87.4176) (width 0.22) (layer F.Cu) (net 3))
 (segment (start 182.2132 87.4176) (end 184.6952 84.9356) (width 0.22) (layer F.Cu) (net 3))
 (segment (start 184.6952 84.9356) (end 184.6952 82.709) (width 0.22) (layer F.Cu) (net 3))
 (segment (start 184.6952 82.709) (end 184.4862 82.5) (width 0.22) (layer F.Cu) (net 3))
 (segment (start 184.4862 82.5) (end 183.9375 82.5) (width 0.22) (layer F.Cu) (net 3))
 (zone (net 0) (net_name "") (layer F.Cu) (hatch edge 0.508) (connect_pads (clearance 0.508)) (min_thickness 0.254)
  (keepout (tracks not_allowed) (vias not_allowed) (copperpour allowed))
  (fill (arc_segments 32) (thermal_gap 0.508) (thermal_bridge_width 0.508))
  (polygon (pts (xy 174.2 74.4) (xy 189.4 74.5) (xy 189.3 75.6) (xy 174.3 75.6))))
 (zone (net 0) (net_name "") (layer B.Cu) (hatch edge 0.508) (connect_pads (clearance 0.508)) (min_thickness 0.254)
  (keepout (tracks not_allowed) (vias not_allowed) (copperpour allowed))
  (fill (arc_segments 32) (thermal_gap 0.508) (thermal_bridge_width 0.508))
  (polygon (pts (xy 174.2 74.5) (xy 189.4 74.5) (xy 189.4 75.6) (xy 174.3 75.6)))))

